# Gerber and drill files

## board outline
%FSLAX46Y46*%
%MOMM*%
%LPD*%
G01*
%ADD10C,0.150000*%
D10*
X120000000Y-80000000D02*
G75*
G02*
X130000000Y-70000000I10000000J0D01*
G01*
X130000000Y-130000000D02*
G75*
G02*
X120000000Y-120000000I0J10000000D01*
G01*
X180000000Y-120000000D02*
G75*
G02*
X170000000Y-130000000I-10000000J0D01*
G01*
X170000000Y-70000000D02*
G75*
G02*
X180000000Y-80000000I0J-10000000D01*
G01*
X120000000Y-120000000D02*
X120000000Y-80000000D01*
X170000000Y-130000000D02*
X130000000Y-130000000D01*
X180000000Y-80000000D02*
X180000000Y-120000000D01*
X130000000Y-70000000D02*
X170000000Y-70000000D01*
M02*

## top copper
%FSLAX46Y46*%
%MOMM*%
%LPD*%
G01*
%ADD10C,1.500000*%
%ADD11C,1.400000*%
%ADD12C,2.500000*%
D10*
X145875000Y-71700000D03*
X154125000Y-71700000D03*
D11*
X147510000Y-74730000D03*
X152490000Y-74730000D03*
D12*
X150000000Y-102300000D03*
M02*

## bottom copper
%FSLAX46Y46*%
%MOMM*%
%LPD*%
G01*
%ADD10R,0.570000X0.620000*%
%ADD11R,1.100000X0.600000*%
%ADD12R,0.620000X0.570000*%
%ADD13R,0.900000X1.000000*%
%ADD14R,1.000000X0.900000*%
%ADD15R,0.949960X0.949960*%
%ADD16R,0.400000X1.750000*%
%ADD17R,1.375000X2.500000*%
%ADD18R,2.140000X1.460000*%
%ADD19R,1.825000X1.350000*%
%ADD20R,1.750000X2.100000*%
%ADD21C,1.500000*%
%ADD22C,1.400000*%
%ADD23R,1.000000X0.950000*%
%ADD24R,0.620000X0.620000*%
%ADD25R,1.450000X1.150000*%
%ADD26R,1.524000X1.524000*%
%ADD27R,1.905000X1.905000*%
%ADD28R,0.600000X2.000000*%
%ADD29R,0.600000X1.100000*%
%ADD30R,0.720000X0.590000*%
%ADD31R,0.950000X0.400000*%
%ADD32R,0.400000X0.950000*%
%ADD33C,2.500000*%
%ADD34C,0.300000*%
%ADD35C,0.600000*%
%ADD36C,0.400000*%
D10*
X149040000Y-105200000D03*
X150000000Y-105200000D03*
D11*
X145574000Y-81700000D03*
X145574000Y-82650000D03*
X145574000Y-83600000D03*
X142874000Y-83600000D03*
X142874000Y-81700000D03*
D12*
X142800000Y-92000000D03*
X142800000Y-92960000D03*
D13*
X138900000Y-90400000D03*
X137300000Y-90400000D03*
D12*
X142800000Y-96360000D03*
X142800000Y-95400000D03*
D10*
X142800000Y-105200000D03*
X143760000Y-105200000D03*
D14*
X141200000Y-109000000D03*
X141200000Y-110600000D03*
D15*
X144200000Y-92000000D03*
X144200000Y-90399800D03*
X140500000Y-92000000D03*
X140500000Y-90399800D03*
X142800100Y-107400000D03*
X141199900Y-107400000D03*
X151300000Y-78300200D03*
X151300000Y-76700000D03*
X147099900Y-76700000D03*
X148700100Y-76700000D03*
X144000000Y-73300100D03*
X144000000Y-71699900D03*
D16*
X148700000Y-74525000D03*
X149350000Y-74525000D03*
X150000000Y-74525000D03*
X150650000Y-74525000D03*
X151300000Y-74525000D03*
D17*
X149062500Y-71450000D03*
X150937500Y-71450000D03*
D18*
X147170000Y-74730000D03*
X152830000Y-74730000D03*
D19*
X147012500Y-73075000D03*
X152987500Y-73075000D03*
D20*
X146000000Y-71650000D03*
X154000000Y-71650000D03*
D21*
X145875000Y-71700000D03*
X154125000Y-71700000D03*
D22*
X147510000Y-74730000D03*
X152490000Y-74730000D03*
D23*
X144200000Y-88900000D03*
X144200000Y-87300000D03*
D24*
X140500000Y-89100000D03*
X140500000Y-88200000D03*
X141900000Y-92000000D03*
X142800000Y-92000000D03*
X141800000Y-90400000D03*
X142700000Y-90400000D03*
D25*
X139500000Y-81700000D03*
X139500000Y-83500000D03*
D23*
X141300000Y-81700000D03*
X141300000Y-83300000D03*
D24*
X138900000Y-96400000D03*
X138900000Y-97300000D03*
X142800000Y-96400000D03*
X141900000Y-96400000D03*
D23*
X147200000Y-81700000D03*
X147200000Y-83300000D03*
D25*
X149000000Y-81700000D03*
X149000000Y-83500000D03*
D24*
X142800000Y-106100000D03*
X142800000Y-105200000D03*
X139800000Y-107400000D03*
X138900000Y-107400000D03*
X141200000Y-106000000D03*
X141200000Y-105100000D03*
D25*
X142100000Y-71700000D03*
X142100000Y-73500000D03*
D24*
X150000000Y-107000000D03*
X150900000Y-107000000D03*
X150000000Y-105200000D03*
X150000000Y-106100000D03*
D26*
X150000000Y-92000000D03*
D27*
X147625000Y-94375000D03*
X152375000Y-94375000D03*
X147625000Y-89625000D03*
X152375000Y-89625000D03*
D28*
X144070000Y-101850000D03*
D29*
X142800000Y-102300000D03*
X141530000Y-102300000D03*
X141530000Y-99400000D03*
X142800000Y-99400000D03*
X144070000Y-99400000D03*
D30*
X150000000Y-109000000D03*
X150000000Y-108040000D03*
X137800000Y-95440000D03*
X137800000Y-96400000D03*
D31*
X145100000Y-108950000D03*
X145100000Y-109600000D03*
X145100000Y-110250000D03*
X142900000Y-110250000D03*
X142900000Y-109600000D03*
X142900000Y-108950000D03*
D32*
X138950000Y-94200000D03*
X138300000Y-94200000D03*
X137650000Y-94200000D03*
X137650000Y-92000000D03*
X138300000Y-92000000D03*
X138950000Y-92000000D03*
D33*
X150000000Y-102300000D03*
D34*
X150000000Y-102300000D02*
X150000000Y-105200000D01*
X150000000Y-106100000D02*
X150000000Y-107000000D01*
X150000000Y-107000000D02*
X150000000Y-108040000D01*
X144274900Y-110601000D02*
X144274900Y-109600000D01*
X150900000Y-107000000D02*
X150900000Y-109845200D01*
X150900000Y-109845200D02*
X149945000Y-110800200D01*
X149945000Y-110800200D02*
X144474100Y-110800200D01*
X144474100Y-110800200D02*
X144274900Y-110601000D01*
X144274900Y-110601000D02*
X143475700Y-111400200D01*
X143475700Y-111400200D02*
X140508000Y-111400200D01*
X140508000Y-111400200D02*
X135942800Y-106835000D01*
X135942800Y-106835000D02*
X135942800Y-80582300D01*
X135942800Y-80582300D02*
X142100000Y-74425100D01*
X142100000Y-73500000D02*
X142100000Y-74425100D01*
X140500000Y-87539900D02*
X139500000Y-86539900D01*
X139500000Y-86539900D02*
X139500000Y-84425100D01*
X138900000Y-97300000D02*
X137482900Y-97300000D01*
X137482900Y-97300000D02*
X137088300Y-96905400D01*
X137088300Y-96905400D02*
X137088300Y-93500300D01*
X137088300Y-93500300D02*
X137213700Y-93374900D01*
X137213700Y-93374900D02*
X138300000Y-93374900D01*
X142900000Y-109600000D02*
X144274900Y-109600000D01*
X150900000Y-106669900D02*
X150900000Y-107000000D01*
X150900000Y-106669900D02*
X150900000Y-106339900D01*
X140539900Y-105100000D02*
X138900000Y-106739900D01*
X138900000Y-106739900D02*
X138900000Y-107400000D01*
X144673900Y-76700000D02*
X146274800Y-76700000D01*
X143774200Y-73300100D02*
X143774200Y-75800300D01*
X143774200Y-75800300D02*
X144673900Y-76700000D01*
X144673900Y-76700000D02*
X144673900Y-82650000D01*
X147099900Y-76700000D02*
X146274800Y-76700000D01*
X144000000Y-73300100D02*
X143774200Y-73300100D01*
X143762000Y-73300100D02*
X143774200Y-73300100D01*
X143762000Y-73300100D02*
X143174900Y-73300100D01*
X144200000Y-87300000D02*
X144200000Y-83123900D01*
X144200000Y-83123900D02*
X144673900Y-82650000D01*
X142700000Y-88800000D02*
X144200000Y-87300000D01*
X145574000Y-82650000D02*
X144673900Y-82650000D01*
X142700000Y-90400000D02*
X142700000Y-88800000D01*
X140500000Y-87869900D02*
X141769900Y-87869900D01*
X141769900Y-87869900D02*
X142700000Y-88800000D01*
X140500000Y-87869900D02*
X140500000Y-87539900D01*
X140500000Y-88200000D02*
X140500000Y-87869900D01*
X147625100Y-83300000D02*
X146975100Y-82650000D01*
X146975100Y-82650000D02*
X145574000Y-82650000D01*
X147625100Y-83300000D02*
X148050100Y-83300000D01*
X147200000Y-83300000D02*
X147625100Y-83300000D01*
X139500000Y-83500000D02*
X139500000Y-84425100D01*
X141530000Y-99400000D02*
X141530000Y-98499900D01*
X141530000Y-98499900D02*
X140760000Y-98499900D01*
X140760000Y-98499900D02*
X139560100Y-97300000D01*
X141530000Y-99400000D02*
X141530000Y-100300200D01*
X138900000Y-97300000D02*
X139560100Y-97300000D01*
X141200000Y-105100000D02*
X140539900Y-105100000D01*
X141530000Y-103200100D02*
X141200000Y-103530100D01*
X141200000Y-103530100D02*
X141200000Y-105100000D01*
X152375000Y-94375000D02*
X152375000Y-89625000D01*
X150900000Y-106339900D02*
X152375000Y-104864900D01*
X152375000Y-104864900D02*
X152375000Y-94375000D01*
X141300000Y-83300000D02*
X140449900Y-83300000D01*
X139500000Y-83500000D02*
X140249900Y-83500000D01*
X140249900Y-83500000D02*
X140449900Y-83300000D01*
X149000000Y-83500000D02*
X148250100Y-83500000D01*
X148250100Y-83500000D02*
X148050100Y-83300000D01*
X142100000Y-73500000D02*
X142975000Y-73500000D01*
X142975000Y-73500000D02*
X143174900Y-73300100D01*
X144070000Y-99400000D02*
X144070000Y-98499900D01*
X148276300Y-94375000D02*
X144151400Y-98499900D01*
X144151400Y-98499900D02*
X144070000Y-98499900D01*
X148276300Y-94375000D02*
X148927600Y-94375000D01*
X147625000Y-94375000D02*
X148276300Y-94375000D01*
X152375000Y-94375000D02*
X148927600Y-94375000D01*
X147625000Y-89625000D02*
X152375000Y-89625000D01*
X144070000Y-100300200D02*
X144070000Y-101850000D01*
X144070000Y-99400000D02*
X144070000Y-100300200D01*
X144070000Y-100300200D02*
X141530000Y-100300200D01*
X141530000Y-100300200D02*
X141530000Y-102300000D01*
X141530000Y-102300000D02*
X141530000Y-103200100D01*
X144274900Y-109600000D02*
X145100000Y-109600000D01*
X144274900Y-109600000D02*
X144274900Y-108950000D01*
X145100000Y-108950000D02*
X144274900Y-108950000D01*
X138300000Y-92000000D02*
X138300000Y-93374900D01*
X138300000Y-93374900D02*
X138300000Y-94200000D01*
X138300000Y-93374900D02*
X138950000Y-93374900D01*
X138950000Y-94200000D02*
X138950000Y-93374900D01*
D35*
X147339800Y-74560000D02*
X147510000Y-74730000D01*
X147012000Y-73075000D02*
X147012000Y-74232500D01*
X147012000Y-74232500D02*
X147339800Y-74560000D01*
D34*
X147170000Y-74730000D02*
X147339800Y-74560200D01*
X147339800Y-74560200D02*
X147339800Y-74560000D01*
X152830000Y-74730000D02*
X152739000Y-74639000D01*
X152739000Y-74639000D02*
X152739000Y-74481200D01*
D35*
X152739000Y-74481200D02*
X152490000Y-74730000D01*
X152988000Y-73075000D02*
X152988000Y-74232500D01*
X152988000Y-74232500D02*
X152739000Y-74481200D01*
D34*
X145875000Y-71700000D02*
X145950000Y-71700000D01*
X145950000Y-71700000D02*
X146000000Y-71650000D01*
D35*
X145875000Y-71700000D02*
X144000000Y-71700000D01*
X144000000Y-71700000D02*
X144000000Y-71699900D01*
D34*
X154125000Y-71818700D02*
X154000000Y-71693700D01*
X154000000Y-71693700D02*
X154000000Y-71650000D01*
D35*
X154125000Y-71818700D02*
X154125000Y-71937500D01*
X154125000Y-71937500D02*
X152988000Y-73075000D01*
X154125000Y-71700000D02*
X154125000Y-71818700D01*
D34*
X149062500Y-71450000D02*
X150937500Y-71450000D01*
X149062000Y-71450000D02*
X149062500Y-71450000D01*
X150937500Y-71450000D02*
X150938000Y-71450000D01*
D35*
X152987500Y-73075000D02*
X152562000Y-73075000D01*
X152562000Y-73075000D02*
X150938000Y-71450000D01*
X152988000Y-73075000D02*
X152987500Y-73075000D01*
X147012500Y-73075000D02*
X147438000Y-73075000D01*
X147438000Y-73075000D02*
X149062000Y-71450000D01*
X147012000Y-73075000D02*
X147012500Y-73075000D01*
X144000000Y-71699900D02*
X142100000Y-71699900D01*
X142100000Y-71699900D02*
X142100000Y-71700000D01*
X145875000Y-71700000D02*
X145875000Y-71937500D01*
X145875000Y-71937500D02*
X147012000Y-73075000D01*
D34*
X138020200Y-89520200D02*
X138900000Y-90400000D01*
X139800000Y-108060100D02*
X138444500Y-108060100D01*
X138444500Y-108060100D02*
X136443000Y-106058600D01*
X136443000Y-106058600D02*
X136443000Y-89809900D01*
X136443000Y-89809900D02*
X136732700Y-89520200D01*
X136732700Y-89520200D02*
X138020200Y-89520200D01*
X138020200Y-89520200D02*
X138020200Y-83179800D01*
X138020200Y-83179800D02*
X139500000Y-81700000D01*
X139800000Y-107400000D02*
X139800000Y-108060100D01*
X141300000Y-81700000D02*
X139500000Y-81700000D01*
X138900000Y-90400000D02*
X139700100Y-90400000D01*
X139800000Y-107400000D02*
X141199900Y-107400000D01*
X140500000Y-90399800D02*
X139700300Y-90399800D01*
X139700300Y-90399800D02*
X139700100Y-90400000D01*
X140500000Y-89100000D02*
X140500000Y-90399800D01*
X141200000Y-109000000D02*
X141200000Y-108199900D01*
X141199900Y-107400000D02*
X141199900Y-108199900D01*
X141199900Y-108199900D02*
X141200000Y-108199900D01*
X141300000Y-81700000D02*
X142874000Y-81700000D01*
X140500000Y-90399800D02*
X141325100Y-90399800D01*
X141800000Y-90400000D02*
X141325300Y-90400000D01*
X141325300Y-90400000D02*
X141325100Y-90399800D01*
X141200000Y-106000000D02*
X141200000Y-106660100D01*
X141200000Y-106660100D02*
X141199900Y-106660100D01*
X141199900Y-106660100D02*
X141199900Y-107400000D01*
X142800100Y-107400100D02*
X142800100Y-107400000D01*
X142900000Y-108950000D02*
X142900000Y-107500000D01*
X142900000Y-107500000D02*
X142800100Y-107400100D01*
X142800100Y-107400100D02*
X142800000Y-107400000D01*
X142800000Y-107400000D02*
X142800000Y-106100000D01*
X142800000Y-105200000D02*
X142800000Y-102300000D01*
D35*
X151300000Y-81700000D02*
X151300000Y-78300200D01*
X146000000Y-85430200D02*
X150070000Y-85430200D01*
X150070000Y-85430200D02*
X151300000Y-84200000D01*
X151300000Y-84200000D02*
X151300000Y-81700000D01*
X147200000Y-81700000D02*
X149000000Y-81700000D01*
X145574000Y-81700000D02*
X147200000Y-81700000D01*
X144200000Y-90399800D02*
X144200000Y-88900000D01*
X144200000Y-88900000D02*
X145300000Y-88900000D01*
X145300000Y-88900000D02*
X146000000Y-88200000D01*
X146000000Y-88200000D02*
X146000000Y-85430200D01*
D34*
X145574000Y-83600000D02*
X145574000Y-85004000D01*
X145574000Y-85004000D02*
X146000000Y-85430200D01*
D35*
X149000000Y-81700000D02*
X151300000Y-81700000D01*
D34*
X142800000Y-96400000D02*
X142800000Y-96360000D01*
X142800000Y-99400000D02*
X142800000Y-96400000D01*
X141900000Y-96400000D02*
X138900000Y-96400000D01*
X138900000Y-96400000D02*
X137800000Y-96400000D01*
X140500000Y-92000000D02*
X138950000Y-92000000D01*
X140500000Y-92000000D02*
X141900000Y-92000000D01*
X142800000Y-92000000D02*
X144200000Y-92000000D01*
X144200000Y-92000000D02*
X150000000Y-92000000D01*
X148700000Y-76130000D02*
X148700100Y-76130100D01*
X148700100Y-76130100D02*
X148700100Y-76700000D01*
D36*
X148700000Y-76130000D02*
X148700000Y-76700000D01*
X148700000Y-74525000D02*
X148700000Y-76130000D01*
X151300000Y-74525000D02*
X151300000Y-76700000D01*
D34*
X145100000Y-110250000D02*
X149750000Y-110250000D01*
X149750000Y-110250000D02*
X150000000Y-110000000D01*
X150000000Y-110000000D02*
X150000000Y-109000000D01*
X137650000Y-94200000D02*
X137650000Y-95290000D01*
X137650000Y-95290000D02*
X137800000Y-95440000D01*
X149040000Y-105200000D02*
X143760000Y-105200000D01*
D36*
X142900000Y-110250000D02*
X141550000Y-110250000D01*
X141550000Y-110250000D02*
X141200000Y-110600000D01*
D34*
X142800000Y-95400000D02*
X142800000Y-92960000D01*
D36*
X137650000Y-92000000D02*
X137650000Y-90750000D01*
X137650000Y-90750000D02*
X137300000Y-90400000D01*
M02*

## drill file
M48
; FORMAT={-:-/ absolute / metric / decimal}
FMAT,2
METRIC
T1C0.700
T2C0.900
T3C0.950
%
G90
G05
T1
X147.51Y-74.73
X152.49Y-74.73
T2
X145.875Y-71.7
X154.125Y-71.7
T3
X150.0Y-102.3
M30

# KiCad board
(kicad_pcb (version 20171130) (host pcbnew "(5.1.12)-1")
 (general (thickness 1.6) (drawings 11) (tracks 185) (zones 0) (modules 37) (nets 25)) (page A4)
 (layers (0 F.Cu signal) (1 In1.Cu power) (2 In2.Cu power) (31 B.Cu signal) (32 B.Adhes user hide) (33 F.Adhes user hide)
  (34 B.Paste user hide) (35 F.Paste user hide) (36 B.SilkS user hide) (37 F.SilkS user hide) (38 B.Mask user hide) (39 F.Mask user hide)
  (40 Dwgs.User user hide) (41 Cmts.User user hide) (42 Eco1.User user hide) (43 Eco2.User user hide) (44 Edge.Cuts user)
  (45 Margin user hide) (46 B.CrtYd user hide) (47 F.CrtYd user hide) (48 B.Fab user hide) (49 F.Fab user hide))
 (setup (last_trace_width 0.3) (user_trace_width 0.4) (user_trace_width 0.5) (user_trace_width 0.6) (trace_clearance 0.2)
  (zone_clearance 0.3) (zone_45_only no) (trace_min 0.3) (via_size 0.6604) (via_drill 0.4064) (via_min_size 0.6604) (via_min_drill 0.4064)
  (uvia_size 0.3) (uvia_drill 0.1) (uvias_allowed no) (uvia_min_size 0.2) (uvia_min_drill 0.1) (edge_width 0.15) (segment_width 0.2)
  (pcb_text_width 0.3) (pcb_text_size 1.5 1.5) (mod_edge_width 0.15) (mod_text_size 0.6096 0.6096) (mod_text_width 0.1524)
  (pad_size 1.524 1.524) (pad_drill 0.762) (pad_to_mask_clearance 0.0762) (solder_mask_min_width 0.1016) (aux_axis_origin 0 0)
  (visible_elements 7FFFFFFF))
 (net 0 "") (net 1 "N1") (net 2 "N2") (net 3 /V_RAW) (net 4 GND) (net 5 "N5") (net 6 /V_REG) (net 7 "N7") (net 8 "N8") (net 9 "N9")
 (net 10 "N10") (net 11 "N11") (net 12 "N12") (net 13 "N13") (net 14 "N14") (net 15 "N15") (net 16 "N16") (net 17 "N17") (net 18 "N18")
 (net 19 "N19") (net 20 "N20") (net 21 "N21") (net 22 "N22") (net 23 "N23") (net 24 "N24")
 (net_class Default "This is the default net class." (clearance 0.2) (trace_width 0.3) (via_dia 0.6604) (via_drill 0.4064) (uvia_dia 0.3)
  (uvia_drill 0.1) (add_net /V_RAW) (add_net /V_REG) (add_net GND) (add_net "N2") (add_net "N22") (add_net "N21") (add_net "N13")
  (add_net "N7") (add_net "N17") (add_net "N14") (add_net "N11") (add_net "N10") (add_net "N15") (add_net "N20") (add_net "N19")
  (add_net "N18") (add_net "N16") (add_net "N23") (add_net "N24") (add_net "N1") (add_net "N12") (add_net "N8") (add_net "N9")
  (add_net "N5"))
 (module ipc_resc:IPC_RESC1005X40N (layer B.Cu) (at 149.52 105.2)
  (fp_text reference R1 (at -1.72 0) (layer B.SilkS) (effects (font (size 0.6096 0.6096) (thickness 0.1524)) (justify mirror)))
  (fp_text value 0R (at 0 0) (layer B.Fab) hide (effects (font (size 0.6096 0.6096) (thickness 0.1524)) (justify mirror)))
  (pad 1 smd rect (at -0.48 0) (size 0.57 0.62) (layers B.Cu B.Paste B.Mask) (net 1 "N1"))
  (pad 2 smd rect (at 0.48 0) (size 0.57 0.62) (layers B.Cu B.Paste B.Mask) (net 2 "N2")))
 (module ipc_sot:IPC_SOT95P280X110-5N (layer B.Cu) (at 144.224 82.65 180)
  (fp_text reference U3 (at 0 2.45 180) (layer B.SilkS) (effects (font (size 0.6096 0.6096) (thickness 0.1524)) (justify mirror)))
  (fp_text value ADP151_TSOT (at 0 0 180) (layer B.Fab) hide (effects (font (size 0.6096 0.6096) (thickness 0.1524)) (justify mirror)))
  (pad 1 smd rect (at -1.35 0.95 180) (size 1.1 0.6) (layers B.Cu B.Paste B.Mask) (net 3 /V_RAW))
  (pad 2 smd rect (at -1.35 0 180) (size 1.1 0.6) (layers B.Cu B.Paste B.Mask) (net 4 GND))
  (pad 3 smd rect (at -1.35 -0.95 180) (size 1.1 0.6) (layers B.Cu B.Paste B.Mask) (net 3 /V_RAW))
  (pad 4 smd rect (at 1.35 -0.95 180) (size 1.1 0.6) (layers B.Cu B.Paste B.Mask) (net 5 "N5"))
  (pad 5 smd rect (at 1.35 0.95 180) (size 1.1 0.6) (layers B.Cu B.Paste B.Mask) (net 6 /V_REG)))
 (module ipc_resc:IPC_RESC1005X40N (layer B.Cu) (at 142.8 92.48 270)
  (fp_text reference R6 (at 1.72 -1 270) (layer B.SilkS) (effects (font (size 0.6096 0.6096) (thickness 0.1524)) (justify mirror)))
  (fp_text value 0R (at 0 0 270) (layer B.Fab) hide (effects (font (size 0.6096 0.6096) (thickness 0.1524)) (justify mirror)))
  (pad 1 smd rect (at -0.48 0 270) (size 0.57 0.62) (layers B.Cu B.Paste B.Mask) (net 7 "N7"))
  (pad 2 smd rect (at 0.48 0 270) (size 0.57 0.62) (layers B.Cu B.Paste B.Mask) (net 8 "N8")))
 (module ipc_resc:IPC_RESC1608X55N (layer B.Cu) (at 138.1 90.4 180)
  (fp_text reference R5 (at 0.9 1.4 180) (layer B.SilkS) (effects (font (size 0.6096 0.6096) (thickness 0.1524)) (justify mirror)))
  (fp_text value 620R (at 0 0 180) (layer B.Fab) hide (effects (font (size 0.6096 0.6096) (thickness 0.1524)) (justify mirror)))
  (pad 1 smd rect (at -0.8 0 180) (size 0.9 1) (layers B.Cu B.Paste B.Mask) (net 6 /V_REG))
  (pad 2 smd rect (at 0.8 0 180) (size 0.9 1) (layers B.Cu B.Paste B.Mask) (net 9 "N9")))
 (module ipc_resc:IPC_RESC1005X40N (layer B.Cu) (at 142.8 95.88 90)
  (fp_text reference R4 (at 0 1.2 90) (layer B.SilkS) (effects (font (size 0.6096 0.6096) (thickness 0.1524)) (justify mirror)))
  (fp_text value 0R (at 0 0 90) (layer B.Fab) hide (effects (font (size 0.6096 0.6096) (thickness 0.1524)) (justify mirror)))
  (pad 1 smd rect (at -0.48 0 90) (size 0.57 0.62) (layers B.Cu B.Paste B.Mask) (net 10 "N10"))
  (pad 2 smd rect (at 0.48 0 90) (size 0.57 0.62) (layers B.Cu B.Paste B.Mask) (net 8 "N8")))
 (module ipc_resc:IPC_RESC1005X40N (layer B.Cu) (at 143.28 105.2)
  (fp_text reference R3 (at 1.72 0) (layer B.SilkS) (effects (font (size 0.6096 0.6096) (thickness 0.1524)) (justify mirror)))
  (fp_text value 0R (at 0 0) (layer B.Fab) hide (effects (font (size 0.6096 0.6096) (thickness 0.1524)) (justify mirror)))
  (pad 1 smd rect (at -0.48 0) (size 0.57 0.62) (layers B.Cu B.Paste B.Mask) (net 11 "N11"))
  (pad 2 smd rect (at 0.48 0) (size 0.57 0.62) (layers B.Cu B.Paste B.Mask) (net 1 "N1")))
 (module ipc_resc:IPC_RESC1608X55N (layer B.Cu) (at 141.2 109.8 270)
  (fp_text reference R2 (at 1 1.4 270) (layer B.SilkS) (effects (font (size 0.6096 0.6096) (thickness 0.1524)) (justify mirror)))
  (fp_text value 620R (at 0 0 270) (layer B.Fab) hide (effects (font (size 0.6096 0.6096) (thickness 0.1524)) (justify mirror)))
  (pad 1 smd rect (at -0.8 0 270) (size 0.9 1) (layers B.Cu B.Paste B.Mask) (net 6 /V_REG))
  (pad 2 smd rect (at 0.8 0 270) (size 0.9 1) (layers B.Cu B.Paste B.Mask) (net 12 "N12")))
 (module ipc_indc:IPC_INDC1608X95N (layer B.Cu) (at 144.2 91.1999 90)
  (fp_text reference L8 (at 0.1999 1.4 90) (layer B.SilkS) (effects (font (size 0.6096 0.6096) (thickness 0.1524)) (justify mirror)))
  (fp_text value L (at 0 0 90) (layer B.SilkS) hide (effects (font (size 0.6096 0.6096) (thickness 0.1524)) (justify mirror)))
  (pad 1 smd rect (at -0.8001 0 90) (size 0.94996 0.94996) (layers B.Cu B.Paste B.Mask) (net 7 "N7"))
  (pad 2 smd rect (at 0.8001 0 90) (size 0.94996 0.94996) (layers B.Cu B.Paste B.Mask) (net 3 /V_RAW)))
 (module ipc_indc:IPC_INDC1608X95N (layer B.Cu) (at 140.5 91.1999 90)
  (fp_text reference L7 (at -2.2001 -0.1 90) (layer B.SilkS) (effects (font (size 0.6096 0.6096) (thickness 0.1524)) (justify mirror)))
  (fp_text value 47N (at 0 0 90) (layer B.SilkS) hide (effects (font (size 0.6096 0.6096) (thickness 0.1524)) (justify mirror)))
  (pad 1 smd rect (at -0.8001 0 90) (size 0.94996 0.94996) (layers B.Cu B.Paste B.Mask) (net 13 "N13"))
  (pad 2 smd rect (at 0.8001 0 90) (size 0.94996 0.94996) (layers B.Cu B.Paste B.Mask) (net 6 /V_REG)))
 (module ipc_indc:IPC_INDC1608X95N (layer B.Cu) (at 142 107.4 180)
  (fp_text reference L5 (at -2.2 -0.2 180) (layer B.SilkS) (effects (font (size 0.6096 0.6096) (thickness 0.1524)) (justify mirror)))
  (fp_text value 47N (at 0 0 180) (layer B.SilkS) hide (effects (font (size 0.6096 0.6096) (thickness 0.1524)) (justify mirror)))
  (pad 1 smd rect (at -0.8001 0 180) (size 0.94996 0.94996) (layers B.Cu B.Paste B.Mask) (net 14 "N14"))
  (pad 2 smd rect (at 0.8001 0 180) (size 0.94996 0.94996) (layers B.Cu B.Paste B.Mask) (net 6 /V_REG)))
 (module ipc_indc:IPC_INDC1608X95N (layer B.Cu) (at 151.3 77.5001 90)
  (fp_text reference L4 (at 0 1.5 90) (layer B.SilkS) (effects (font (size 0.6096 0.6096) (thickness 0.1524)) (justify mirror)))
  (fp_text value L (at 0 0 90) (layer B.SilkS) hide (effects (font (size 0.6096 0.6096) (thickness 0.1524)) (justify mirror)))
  (pad 1 smd rect (at -0.8001 0 90) (size 0.94996 0.94996) (layers B.Cu B.Paste B.Mask) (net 3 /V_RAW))
  (pad 2 smd rect (at 0.8001 0 90) (size 0.94996 0.94996) (layers B.Cu B.Paste B.Mask) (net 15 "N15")))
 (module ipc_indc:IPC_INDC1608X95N (layer B.Cu) (at 147.9 76.7)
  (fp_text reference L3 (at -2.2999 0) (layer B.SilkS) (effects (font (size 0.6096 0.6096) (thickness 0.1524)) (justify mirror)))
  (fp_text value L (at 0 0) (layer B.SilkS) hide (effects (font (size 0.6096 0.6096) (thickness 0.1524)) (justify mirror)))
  (pad 1 smd rect (at -0.8001 0) (size 0.94996 0.94996) (layers B.Cu B.Paste B.Mask) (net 4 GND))
  (pad 2 smd rect (at 0.8001 0) (size 0.94996 0.94996) (layers B.Cu B.Paste B.Mask) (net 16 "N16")))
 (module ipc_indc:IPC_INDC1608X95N (layer B.Cu) (at 144 72.5 90)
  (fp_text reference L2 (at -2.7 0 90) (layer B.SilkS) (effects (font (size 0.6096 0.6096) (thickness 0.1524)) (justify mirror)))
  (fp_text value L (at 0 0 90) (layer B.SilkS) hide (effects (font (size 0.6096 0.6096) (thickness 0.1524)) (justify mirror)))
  (pad 1 smd rect (at -0.8001 0 90) (size 0.94996 0.94996) (layers B.Cu B.Paste B.Mask) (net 4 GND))
  (pad 2 smd rect (at 0.8001 0 90) (size 0.94996 0.94996) (layers B.Cu B.Paste B.Mask) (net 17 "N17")))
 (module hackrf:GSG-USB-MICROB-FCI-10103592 (layer B.Cu) (at 150 70 270)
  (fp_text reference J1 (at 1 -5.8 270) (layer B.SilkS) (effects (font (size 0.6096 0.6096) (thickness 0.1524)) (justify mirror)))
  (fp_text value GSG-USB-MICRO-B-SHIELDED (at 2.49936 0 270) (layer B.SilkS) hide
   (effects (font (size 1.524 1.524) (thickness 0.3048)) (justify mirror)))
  (pad 5 smd rect (at 4.525 1.3 270) (size 1.75 0.4) (layers B.Cu B.Paste B.Mask) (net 16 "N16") (solder_mask_margin 0.1016)
   (clearance 0.2032))
  (pad 4 smd rect (at 4.525 0.65 270) (size 1.75 0.4) (layers B.Cu B.Paste B.Mask) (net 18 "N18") (solder_mask_margin 0.1016)
   (clearance 0.2032))
  (pad 3 smd rect (at 4.525 0 270) (size 1.75 0.4) (layers B.Cu B.Paste B.Mask) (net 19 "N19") (solder_mask_margin 0.1016)
   (clearance 0.2032))
  (pad 2 smd rect (at 4.525 -0.65 270) (size 1.75 0.4) (layers B.Cu B.Paste B.Mask) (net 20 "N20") (solder_mask_margin 0.1016)
   (clearance 0.2032))
  (pad 1 smd rect (at 4.525 -1.3 270) (size 1.75 0.4) (layers B.Cu B.Paste B.Mask) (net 15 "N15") (solder_mask_margin 0.1016)
   (clearance 0.2032))
  (pad 0 smd rect (at 1.45 0.9375 270) (size 2.5 1.375) (layers B.Cu B.Paste B.Mask) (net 17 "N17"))
  (pad 0 smd rect (at 1.45 -0.9375 270) (size 2.5 1.375) (layers B.Cu B.Paste B.Mask) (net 17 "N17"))
  (pad 0 smd rect (at 4.73 2.83 270) (size 1.46 2.14) (layers B.Cu B.Paste B.Mask) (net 17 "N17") (solder_paste_margin_ratio -0.05))
  (pad 0 smd rect (at 4.73 -2.83 270) (size 1.46 2.14) (layers B.Cu B.Paste B.Mask) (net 17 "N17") (solder_paste_margin_ratio -0.05))
  (pad 0 smd rect (at 3.075 2.9875 270) (size 1.35 1.825) (layers B.Cu B.Mask) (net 17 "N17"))
  (pad 0 smd rect (at 3.075 -2.9875 270) (size 1.35 1.825) (layers B.Cu B.Mask) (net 17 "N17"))
  (pad 0 smd rect (at 1.65 4 270) (size 2.1 1.75) (layers B.Cu B.Paste B.Mask) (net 17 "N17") (solder_paste_margin_ratio -0.05))
  (pad 0 smd rect (at 1.65 -4 270) (size 2.1 1.75) (layers B.Cu B.Paste B.Mask) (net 17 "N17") (solder_paste_margin_ratio -0.05))
  (pad 0 thru_hole circle (at 1.7 4.125 270) (size 1.5 1.5) (drill 0.9) (layers *.Cu *.Mask) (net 17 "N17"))
  (pad 0 thru_hole circle (at 1.7 -4.125 270) (size 1.5 1.5) (drill 0.9) (layers *.Cu *.Mask) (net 17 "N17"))
  (pad 0 thru_hole circle (at 4.73 2.49 270) (size 1.4 1.4) (drill 0.7) (layers *.Cu *.Mask) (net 17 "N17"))
  (pad 0 thru_hole circle (at 4.73 -2.49 270) (size 1.4 1.4) (drill 0.7) (layers *.Cu *.Mask) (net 17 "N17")))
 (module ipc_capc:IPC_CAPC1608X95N (layer B.Cu) (at 144.2 88.1 90)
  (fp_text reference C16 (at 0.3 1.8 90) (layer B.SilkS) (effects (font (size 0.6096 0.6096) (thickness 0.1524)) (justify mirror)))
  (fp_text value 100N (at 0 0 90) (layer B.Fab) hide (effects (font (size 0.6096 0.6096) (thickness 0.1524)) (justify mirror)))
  (pad 1 smd rect (at -0.8 0 90) (size 0.95 1) (layers B.Cu B.Paste B.Mask) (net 3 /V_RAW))
  (pad 2 smd rect (at 0.8 0 90) (size 0.95 1) (layers B.Cu B.Paste B.Mask) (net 4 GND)))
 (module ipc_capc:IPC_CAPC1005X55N (layer B.Cu) (at 140.5 88.65 90)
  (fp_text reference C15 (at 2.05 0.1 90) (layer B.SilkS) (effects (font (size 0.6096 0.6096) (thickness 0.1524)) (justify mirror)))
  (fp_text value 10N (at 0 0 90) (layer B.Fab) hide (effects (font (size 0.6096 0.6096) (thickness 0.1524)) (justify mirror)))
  (pad 1 smd rect (at -0.45 0 90) (size 0.62 0.62) (layers B.Cu B.Paste B.Mask) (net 6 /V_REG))
  (pad 2 smd rect (at 0.45 0 90) (size 0.62 0.62) (layers B.Cu B.Paste B.Mask) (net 4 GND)))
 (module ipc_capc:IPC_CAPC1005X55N (layer B.Cu) (at 142.35 92)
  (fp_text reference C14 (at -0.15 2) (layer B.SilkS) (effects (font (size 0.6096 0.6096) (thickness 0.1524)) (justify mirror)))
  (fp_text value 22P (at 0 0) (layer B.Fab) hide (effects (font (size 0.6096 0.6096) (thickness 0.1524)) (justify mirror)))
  (pad 1 smd rect (at -0.45 0) (size 0.62 0.62) (layers B.Cu B.Paste B.Mask) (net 13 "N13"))
  (pad 2 smd rect (at 0.45 0) (size 0.62 0.62) (layers B.Cu B.Paste B.Mask) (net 7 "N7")))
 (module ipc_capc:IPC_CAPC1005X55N (layer B.Cu) (at 142.25 90.4)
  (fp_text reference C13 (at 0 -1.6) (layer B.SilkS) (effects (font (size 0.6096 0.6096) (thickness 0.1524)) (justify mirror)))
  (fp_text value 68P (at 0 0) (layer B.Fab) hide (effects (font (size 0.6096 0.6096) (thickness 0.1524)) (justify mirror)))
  (pad 1 smd rect (at -0.45 0) (size 0.62 0.62) (layers B.Cu B.Paste B.Mask) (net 6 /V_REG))
  (pad 2 smd rect (at 0.45 0) (size 0.62 0.62) (layers B.Cu B.Paste B.Mask) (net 4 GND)))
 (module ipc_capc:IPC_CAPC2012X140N (layer B.Cu) (at 139.5 82.6 270)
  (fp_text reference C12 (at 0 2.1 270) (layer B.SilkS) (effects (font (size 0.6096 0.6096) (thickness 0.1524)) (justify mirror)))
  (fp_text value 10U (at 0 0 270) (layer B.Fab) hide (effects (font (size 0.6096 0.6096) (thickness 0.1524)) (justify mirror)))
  (pad 1 smd rect (at -0.9 0 270) (size 1.15 1.45) (layers B.Cu B.Paste B.Mask) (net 6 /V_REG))
  (pad 2 smd rect (at 0.9 0 270) (size 1.15 1.45) (layers B.Cu B.Paste B.Mask) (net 4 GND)))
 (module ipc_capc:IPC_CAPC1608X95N (layer B.Cu) (at 141.3 82.5 270)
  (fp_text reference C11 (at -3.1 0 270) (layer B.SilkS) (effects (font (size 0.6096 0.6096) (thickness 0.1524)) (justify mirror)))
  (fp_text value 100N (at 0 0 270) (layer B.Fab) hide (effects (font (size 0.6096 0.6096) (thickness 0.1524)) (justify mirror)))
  (pad 1 smd rect (at -0.8 0 270) (size 0.95 1) (layers B.Cu B.Paste B.Mask) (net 6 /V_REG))
  (pad 2 smd rect (at 0.8 0 270) (size 0.95 1) (layers B.Cu B.Paste B.Mask) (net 4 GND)))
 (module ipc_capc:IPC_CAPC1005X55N (layer B.Cu) (at 138.9 96.85 270)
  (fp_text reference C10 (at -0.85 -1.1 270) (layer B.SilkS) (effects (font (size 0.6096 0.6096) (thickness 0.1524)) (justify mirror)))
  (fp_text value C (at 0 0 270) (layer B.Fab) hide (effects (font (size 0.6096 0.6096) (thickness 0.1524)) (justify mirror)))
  (pad 1 smd rect (at -0.45 0 270) (size 0.62 0.62) (layers B.Cu B.Paste B.Mask) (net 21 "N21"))
  (pad 2 smd rect (at 0.45 0 270) (size 0.62 0.62) (layers B.Cu B.Paste B.Mask) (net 4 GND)))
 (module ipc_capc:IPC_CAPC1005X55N (layer B.Cu) (at 142.35 96.4 180)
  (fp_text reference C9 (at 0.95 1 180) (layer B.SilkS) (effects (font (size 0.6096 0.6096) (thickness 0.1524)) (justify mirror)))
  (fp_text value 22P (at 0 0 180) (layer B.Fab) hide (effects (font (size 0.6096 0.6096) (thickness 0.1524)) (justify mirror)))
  (pad 1 smd rect (at -0.45 0 180) (size 0.62 0.62) (layers B.Cu B.Paste B.Mask) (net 10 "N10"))
  (pad 2 smd rect (at 0.45 0 180) (size 0.62 0.62) (layers B.Cu B.Paste B.Mask) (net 21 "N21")))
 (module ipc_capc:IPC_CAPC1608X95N (layer B.Cu) (at 147.2 82.5 270)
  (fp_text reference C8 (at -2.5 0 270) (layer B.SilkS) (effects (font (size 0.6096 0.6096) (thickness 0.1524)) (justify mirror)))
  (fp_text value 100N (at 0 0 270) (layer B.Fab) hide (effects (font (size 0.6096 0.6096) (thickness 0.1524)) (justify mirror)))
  (pad 1 smd rect (at -0.8 0 270) (size 0.95 1) (layers B.Cu B.Paste B.Mask) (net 3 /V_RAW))
  (pad 2 smd rect (at 0.8 0 270) (size 0.95 1) (layers B.Cu B.Paste B.Mask) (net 4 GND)))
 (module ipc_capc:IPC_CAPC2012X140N (layer B.Cu) (at 149 82.6 270)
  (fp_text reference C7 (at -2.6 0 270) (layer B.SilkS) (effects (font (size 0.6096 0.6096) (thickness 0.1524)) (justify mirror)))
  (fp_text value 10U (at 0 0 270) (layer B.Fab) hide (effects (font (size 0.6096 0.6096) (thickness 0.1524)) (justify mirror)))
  (pad 1 smd rect (at -0.9 0 270) (size 1.15 1.45) (layers B.Cu B.Paste B.Mask) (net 3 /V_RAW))
  (pad 2 smd rect (at 0.9 0 270) (size 1.15 1.45) (layers B.Cu B.Paste B.Mask) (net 4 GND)))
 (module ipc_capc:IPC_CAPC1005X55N (layer B.Cu) (at 142.8 105.65 90)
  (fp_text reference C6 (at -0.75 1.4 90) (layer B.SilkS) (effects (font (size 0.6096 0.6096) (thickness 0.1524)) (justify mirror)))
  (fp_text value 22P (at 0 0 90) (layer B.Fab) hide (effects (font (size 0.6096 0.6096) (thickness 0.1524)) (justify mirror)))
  (pad 1 smd rect (at -0.45 0 90) (size 0.62 0.62) (layers B.Cu B.Paste B.Mask) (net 14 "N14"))
  (pad 2 smd rect (at 0.45 0 90) (size 0.62 0.62) (layers B.Cu B.Paste B.Mask) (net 11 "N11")))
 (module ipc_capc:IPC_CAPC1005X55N (layer B.Cu) (at 139.35 107.4 180)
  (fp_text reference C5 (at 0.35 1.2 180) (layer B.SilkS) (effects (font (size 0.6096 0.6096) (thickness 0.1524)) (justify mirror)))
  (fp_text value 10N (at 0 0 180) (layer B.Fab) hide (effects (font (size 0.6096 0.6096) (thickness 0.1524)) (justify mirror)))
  (pad 1 smd rect (at -0.45 0 180) (size 0.62 0.62) (layers B.Cu B.Paste B.Mask) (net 6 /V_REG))
  (pad 2 smd rect (at 0.45 0 180) (size 0.62 0.62) (layers B.Cu B.Paste B.Mask) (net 4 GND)))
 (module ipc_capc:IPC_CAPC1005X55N (layer B.Cu) (at 141.2 105.55 90)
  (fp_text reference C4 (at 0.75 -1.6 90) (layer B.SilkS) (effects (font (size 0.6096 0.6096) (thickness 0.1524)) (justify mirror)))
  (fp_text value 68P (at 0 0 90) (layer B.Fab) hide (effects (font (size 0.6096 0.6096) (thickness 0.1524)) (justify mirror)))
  (pad 1 smd rect (at -0.45 0 90) (size 0.62 0.62) (layers B.Cu B.Paste B.Mask) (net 6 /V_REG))
  (pad 2 smd rect (at 0.45 0 90) (size 0.62 0.62) (layers B.Cu B.Paste B.Mask) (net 4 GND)))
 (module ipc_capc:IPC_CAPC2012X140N (layer B.Cu) (at 142.1 72.6 270)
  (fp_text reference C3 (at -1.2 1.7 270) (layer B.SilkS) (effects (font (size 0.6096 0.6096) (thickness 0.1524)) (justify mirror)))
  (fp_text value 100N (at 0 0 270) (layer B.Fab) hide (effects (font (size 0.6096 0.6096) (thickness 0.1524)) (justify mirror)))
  (pad 1 smd rect (at -0.9 0 270) (size 1.15 1.45) (layers B.Cu B.Paste B.Mask) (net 17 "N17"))
  (pad 2 smd rect (at 0.9 0 270) (size 1.15 1.45) (layers B.Cu B.Paste B.Mask) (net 4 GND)))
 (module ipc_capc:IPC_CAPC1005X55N (layer B.Cu) (at 150.45 107)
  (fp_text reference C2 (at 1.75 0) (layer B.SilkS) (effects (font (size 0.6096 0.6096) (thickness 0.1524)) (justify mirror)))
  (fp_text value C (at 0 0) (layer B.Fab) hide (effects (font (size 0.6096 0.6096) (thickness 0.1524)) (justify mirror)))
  (pad 1 smd rect (at -0.45 0) (size 0.62 0.62) (layers B.Cu B.Paste B.Mask) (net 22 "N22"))
  (pad 2 smd rect (at 0.45 0) (size 0.62 0.62) (layers B.Cu B.Paste B.Mask) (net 4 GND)))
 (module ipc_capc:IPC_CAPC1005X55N (layer B.Cu) (at 150 105.65 270)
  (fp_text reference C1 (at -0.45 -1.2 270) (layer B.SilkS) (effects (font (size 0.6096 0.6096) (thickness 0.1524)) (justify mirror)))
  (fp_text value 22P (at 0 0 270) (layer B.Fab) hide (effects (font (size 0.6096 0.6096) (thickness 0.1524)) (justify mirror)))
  (pad 1 smd rect (at -0.45 0 270) (size 0.62 0.62) (layers B.Cu B.Paste B.Mask) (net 2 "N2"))
  (pad 2 smd rect (at 0.45 0 270) (size 0.62 0.62) (layers B.Cu B.Paste B.Mask) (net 22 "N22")))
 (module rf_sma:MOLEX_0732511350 (layer B.Cu) (at 150 92)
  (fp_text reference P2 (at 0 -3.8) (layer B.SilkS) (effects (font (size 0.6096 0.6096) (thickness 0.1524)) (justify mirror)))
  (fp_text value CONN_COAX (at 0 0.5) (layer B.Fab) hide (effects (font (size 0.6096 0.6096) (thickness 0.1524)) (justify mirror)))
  (pad 1 smd rect (at 0 0) (size 1.524 1.524) (layers B.Cu B.Paste B.Mask) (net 7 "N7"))
  (pad 2 smd rect (at -2.375 2.375) (size 1.905 1.905) (layers B.Cu B.Paste B.Mask) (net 4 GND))
  (pad 2 smd rect (at 2.375 2.375) (size 1.905 1.905) (layers B.Cu B.Paste B.Mask) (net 4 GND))
  (pad 2 smd rect (at -2.375 -2.375) (size 1.905 1.905) (layers B.Cu B.Paste B.Mask) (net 4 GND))
  (pad 2 smd rect (at 2.375 -2.375) (size 1.905 1.905) (layers B.Cu B.Paste B.Mask) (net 4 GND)))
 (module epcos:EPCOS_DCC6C (layer B.Cu) (at 142.8 100.85 90)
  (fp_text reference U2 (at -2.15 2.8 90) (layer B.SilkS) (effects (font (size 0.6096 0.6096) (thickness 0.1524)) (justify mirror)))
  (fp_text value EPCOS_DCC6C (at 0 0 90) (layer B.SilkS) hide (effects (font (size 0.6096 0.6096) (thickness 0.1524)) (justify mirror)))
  (pad 1 smd rect (at -1 1.27 90) (size 2 0.6) (layers B.Cu B.Paste B.Mask) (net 4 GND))
  (pad 2 smd rect (at -1.45 0 90) (size 1.1 0.6) (layers B.Cu B.Paste B.Mask) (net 11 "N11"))
  (pad 3 smd rect (at -1.45 -1.27 90) (size 1.1 0.6) (layers B.Cu B.Paste B.Mask) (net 4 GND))
  (pad 4 smd rect (at 1.45 -1.27 90) (size 1.1 0.6) (layers B.Cu B.Paste B.Mask) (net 4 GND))
  (pad 5 smd rect (at 1.45 0 90) (size 1.1 0.6) (layers B.Cu B.Paste B.Mask) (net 10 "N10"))
  (pad 6 smd rect (at 1.45 1.27 90) (size 1.1 0.6) (layers B.Cu B.Paste B.Mask) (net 4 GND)))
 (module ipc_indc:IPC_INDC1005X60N (layer B.Cu) (at 150 108.52 90)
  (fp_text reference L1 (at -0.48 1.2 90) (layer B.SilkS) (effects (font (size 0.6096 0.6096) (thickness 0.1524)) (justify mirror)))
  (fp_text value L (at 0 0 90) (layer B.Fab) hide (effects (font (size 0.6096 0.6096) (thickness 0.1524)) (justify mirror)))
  (pad 1 smd rect (at -0.48 0 90) (size 0.59 0.72) (layers B.Cu B.Paste B.Mask) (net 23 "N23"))
  (pad 2 smd rect (at 0.48 0 90) (size 0.59 0.72) (layers B.Cu B.Paste B.Mask) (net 22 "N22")))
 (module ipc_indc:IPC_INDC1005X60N (layer B.Cu) (at 137.8 95.92 270)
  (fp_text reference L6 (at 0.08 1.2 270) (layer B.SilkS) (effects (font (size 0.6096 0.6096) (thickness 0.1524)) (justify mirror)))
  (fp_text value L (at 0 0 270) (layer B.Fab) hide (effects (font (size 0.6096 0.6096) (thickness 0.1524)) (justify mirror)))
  (pad 1 smd rect (at -0.48 0 270) (size 0.59 0.72) (layers B.Cu B.Paste B.Mask) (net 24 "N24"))
  (pad 2 smd rect (at 0.48 0 270) (size 0.59 0.72) (layers B.Cu B.Paste B.Mask) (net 21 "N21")))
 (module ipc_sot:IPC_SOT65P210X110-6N (layer B.Cu) (at 144 109.6 180)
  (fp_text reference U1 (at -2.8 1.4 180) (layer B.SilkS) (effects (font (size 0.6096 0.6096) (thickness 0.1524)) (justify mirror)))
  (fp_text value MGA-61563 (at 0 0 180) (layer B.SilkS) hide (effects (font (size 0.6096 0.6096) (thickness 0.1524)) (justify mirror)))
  (pad 1 smd rect (at -1.1 0.65 180) (size 0.95 0.4) (layers B.Cu B.Paste B.Mask) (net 4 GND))
  (pad 2 smd rect (at -1.1 0 180) (size 0.95 0.4) (layers B.Cu B.Paste B.Mask) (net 4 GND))
  (pad 3 smd rect (at -1.1 -0.65 180) (size 0.95 0.4) (layers B.Cu B.Paste B.Mask) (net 23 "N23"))
  (pad 4 smd rect (at 1.1 -0.65 180) (size 0.95 0.4) (layers B.Cu B.Paste B.Mask) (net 12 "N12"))
  (pad 5 smd rect (at 1.1 0 180) (size 0.95 0.4) (layers B.Cu B.Paste B.Mask) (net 4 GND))
  (pad 6 smd rect (at 1.1 0.65 180) (size 0.95 0.4) (layers B.Cu B.Paste B.Mask) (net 14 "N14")))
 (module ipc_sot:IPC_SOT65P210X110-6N (layer B.Cu) (at 138.3 93.1 90)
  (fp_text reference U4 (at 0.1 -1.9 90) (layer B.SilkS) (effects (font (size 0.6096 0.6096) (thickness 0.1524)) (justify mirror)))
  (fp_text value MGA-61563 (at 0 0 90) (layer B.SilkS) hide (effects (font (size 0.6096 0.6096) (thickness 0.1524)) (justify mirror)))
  (pad 1 smd rect (at -1.1 0.65 90) (size 0.95 0.4) (layers B.Cu B.Paste B.Mask) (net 4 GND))
  (pad 2 smd rect (at -1.1 0 90) (size 0.95 0.4) (layers B.Cu B.Paste B.Mask) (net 4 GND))
  (pad 3 smd rect (at -1.1 -0.65 90) (size 0.95 0.4) (layers B.Cu B.Paste B.Mask) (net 24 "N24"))
  (pad 4 smd rect (at 1.1 -0.65 90) (size 0.95 0.4) (layers B.Cu B.Paste B.Mask) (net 9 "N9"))
  (pad 5 smd rect (at 1.1 0 90) (size 0.95 0.4) (layers B.Cu B.Paste B.Mask) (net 4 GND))
  (pad 6 smd rect (at 1.1 0.65 90) (size 0.95 0.4) (layers B.Cu B.Paste B.Mask) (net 13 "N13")))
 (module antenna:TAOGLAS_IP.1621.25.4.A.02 (layer F.Cu) (at 150 100)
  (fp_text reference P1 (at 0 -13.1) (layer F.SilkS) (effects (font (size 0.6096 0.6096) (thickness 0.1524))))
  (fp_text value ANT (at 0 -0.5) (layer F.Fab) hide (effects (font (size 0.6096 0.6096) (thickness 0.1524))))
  (pad 1 thru_hole circle (at 0 2.3) (size 2.5 2.5) (drill 0.95) (layers B.Cu) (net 2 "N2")))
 (gr_arc (start 130 80) (end 120 80) (angle 90) (layer Edge.Cuts) (width 0.15))
 (gr_arc (start 130 120) (end 130 130) (angle 90) (layer Edge.Cuts) (width 0.15))
 (gr_arc (start 170 120) (end 180 120) (angle 90) (layer Edge.Cuts) (width 0.15))
 (gr_arc (start 170 80) (end 170 70) (angle 90) (layer Edge.Cuts) (width 0.15))
 (gr_line (start 120 120) (end 120 80) (layer Edge.Cuts) (width 0.15))
 (gr_line (start 170 130) (end 130 130) (layer Edge.Cuts) (width 0.15))
 (gr_line (start 180 80) (end 180 120) (layer Edge.Cuts) (width 0.15))
 (gr_line (start 130 70) (end 170 70) (layer Edge.Cuts) (width 0.15))
 (segment (start 150 102.3) (end 150 105.2) (width 0.3) (layer B.Cu) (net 2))
 (segment (start 150 106.1) (end 150 107) (width 0.3) (layer B.Cu) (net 22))
 (segment (start 150 107) (end 150 108.04) (width 0.3) (layer B.Cu) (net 22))
 (segment (start 144.2749 110.601) (end 144.2749 109.6) (width 0.3) (layer B.Cu) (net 4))
 (segment (start 150.9 107) (end 150.9 109.8452) (width 0.3) (layer B.Cu) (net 4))
 (segment (start 150.9 109.8452) (end 149.945 110.8002) (width 0.3) (layer B.Cu) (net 4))
 (segment (start 149.945 110.8002) (end 144.4741 110.8002) (width 0.3) (layer B.Cu) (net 4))
 (segment (start 144.4741 110.8002) (end 144.2749 110.601) (width 0.3) (layer B.Cu) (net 4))
 (segment (start 144.2749 110.601) (end 143.4757 111.4002) (width 0.3) (layer B.Cu) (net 4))
 (segment (start 143.4757 111.4002) (end 140.508 111.4002) (width 0.3) (layer B.Cu) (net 4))
 (segment (start 140.508 111.4002) (end 135.9428 106.835) (width 0.3) (layer B.Cu) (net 4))
 (segment (start 135.9428 106.835) (end 135.9428 80.5823) (width 0.3) (layer B.Cu) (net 4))
 (segment (start 135.9428 80.5823) (end 142.1 74.4251) (width 0.3) (layer B.Cu) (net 4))
 (segment (start 142.1 73.5) (end 142.1 74.4251) (width 0.3) (layer B.Cu) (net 4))
 (segment (start 140.5 87.5399) (end 139.5 86.5399) (width 0.3) (layer B.Cu) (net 4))
 (segment (start 139.5 86.5399) (end 139.5 84.4251) (width 0.3) (layer B.Cu) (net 4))
 (segment (start 138.9 97.3) (end 137.4829 97.3) (width 0.3) (layer B.Cu) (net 4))
 (segment (start 137.4829 97.3) (end 137.0883 96.9054) (width 0.3) (layer B.Cu) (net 4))
 (segment (start 137.0883 96.9054) (end 137.0883 93.5003) (width 0.3) (layer B.Cu) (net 4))
 (segment (start 137.0883 93.5003) (end 137.2137 93.3749) (width 0.3) (layer B.Cu) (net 4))
 (segment (start 137.2137 93.3749) (end 138.3 93.3749) (width 0.3) (layer B.Cu) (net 4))
 (segment (start 142.9 109.6) (end 144.2749 109.6) (width 0.3) (layer B.Cu) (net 4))
 (segment (start 150.9 106.6699) (end 150.9 107) (width 0.3) (layer B.Cu) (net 4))
 (segment (start 150.9 106.6699) (end 150.9 106.3399) (width 0.3) (layer B.Cu) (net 4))
 (segment (start 140.5399 105.1) (end 138.9 106.7399) (width 0.3) (layer B.Cu) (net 4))
 (segment (start 138.9 106.7399) (end 138.9 107.4) (width 0.3) (layer B.Cu) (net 4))
 (segment (start 144.6739 76.7) (end 146.2748 76.7) (width 0.3) (layer B.Cu) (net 4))
 (segment (start 143.7742 73.3001) (end 143.7742 75.8003) (width 0.3) (layer B.Cu) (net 4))
 (segment (start 143.7742 75.8003) (end 144.6739 76.7) (width 0.3) (layer B.Cu) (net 4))
 (segment (start 144.6739 76.7) (end 144.6739 82.65) (width 0.3) (layer B.Cu) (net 4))
 (segment (start 147.0999 76.7) (end 146.2748 76.7) (width 0.3) (layer B.Cu) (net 4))
 (segment (start 144 73.3001) (end 143.7742 73.3001) (width 0.3) (layer B.Cu) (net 4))
 (segment (start 143.762 73.3001) (end 143.7742 73.3001) (width 0.3) (layer B.Cu) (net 4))
 (segment (start 143.762 73.3001) (end 143.1749 73.3001) (width 0.3) (layer B.Cu) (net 4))
 (segment (start 144.2 87.3) (end 144.2 83.1239) (width 0.3) (layer B.Cu) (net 4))
 (segment (start 144.2 83.1239) (end 144.6739 82.65) (width 0.3) (layer B.Cu) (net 4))
 (segment (start 142.7 88.8) (end 144.2 87.3) (width 0.3) (layer B.Cu) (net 4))
 (segment (start 145.574 82.65) (end 144.6739 82.65) (width 0.3) (layer B.Cu) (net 4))
 (segment (start 142.7 90.4) (end 142.7 88.8) (width 0.3) (layer B.Cu) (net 4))
 (segment (start 140.5 87.8699) (end 141.7699 87.8699) (width 0.3) (layer B.Cu) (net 4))
 (segment (start 141.7699 87.8699) (end 142.7 88.8) (width 0.3) (layer B.Cu) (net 4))
 (segment (start 140.5 87.8699) (end 140.5 87.5399) (width 0.3) (layer B.Cu) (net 4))
 (segment (start 140.5 88.2) (end 140.5 87.8699) (width 0.3) (layer B.Cu) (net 4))
 (segment (start 147.6251 83.3) (end 146.9751 82.65) (width 0.3) (layer B.Cu) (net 4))
 (segment (start 146.9751 82.65) (end 145.574 82.65) (width 0.3) (layer B.Cu) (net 4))
 (segment (start 147.6251 83.3) (end 148.0501 83.3) (width 0.3) (layer B.Cu) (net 4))
 (segment (start 147.2 83.3) (end 147.6251 83.3) (width 0.3) (layer B.Cu) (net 4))
 (segment (start 139.5 83.5) (end 139.5 84.4251) (width 0.3) (layer B.Cu) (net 4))
 (segment (start 141.53 99.4) (end 141.53 98.4999) (width 0.3) (layer B.Cu) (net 4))
 (segment (start 141.53 98.4999) (end 140.76 98.4999) (width 0.3) (layer B.Cu) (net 4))
 (segment (start 140.76 98.4999) (end 139.5601 97.3) (width 0.3) (layer B.Cu) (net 4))
 (segment (start 141.53 99.4) (end 141.53 100.3002) (width 0.3) (layer B.Cu) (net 4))
 (segment (start 138.9 97.3) (end 139.5601 97.3) (width 0.3) (layer B.Cu) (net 4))
 (segment (start 141.2 105.1) (end 140.5399 105.1) (width 0.3) (layer B.Cu) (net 4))
 (segment (start 141.53 103.2001) (end 141.2 103.5301) (width 0.3) (layer B.Cu) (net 4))
 (segment (start 141.2 103.5301) (end 141.2 105.1) (width 0.3) (layer B.Cu) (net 4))
 (segment (start 152.375 94.375) (end 152.375 89.625) (width 0.3) (layer B.Cu) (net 4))
 (segment (start 150.9 106.3399) (end 152.375 104.8649) (width 0.3) (layer B.Cu) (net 4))
 (segment (start 152.375 104.8649) (end 152.375 94.375) (width 0.3) (layer B.Cu) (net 4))
 (segment (start 141.3 83.3) (end 140.4499 83.3) (width 0.3) (layer B.Cu) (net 4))
 (segment (start 139.5 83.5) (end 140.2499 83.5) (width 0.3) (layer B.Cu) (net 4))
 (segment (start 140.2499 83.5) (end 140.4499 83.3) (width 0.3) (layer B.Cu) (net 4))
 (segment (start 149 83.5) (end 148.2501 83.5) (width 0.3) (layer B.Cu) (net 4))
 (segment (start 148.2501 83.5) (end 148.0501 83.3) (width 0.3) (layer B.Cu) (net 4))
 (segment (start 142.1 73.5) (end 142.975 73.5) (width 0.3) (layer B.Cu) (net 4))
 (segment (start 142.975 73.5) (end 143.1749 73.3001) (width 0.3) (layer B.Cu) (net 4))
 (segment (start 144.07 99.4) (end 144.07 98.4999) (width 0.3) (layer B.Cu) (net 4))
 (segment (start 148.2763 94.375) (end 144.1514 98.4999) (width 0.3) (layer B.Cu) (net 4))
 (segment (start 144.1514 98.4999) (end 144.07 98.4999) (width 0.3) (layer B.Cu) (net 4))
 (segment (start 148.2763 94.375) (end 148.9276 94.375) (width 0.3) (layer B.Cu) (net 4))
 (segment (start 147.625 94.375) (end 148.2763 94.375) (width 0.3) (layer B.Cu) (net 4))
 (segment (start 152.375 94.375) (end 148.9276 94.375) (width 0.3) (layer B.Cu) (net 4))
 (segment (start 147.625 89.625) (end 152.375 89.625) (width 0.3) (layer B.Cu) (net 4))
 (segment (start 144.07 100.3002) (end 144.07 101.85) (width 0.3) (layer B.Cu) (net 4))
 (segment (start 144.07 99.4) (end 144.07 100.3002) (width 0.3) (layer B.Cu) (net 4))
 (segment (start 144.07 100.3002) (end 141.53 100.3002) (width 0.3) (layer B.Cu) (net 4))
 (segment (start 141.53 100.3002) (end 141.53 102.3) (width 0.3) (layer B.Cu) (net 4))
 (segment (start 141.53 102.3) (end 141.53 103.2001) (width 0.3) (layer B.Cu) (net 4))
 (segment (start 144.2749 109.6) (end 145.1 109.6) (width 0.3) (layer B.Cu) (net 4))
 (segment (start 144.2749 109.6) (end 144.2749 108.95) (width 0.3) (layer B.Cu) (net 4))
 (segment (start 145.1 108.95) (end 144.2749 108.95) (width 0.3) (layer B.Cu) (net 4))
 (segment (start 138.3 92) (end 138.3 93.3749) (width 0.3) (layer B.Cu) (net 4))
 (segment (start 138.3 93.3749) (end 138.3 94.2) (width 0.3) (layer B.Cu) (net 4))
 (segment (start 138.3 93.3749) (end 138.95 93.3749) (width 0.3) (layer B.Cu) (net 4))
 (segment (start 138.95 94.2) (end 138.95 93.3749) (width 0.3) (layer B.Cu) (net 4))
 (segment (start 147.3398 74.56) (end 147.51 74.73) (width 0.6) (layer B.Cu) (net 17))
 (segment (start 147.012 73.075) (end 147.012 74.2325) (width 0.6) (layer B.Cu) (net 17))
 (segment (start 147.012 74.2325) (end 147.3398 74.56) (width 0.6) (layer B.Cu) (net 17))
 (segment (start 147.17 74.73) (end 147.3398 74.5602) (width 0.3) (layer B.Cu) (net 17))
 (segment (start 147.3398 74.5602) (end 147.3398 74.56) (width 0.3) (layer B.Cu) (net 17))
 (segment (start 152.83 74.73) (end 152.739 74.639) (width 0.3) (layer B.Cu) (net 17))
 (segment (start 152.739 74.639) (end 152.739 74.4812) (width 0.3) (layer B.Cu) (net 17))
 (segment (start 152.739 74.4812) (end 152.49 74.73) (width 0.6) (layer B.Cu) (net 17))
 (segment (start 152.988 73.075) (end 152.988 74.2325) (width 0.6) (layer B.Cu) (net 17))
 (segment (start 152.988 74.2325) (end 152.739 74.4812) (width 0.6) (layer B.Cu) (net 17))
 (segment (start 145.875 71.7) (end 145.95 71.7) (width 0.3) (layer B.Cu) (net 17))
 (segment (start 145.95 71.7) (end 146 71.65) (width 0.3) (layer B.Cu) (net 17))
 (segment (start 145.875 71.7) (end 144 71.7) (width 0.6) (layer B.Cu) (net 17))
 (segment (start 144 71.7) (end 144 71.6999) (width 0.6) (layer B.Cu) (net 17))
 (segment (start 154.125 71.8187) (end 154 71.6937) (width 0.3) (layer B.Cu) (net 17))
 (segment (start 154 71.6937) (end 154 71.65) (width 0.3) (layer B.Cu) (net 17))
 (segment (start 154.125 71.8187) (end 154.125 71.9375) (width 0.6) (layer B.Cu) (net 17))
 (segment (start 154.125 71.9375) (end 152.988 73.075) (width 0.6) (layer B.Cu) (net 17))
 (segment (start 154.125 71.7) (end 154.125 71.8187) (width 0.6) (layer B.Cu) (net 17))
 (segment (start 149.0625 71.45) (end 150.9375 71.45) (width 0.3) (layer B.Cu) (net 17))
 (segment (start 149.062 71.45) (end 149.0625 71.45) (width 0.3) (layer B.Cu) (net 17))
 (segment (start 150.9375 71.45) (end 150.938 71.45) (width 0.3) (layer B.Cu) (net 17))
 (segment (start 152.9875 73.075) (end 152.562 73.075) (width 0.6) (layer B.Cu) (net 17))
 (segment (start 152.562 73.075) (end 150.938 71.45) (width 0.6) (layer B.Cu) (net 17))
 (segment (start 152.988 73.075) (end 152.9875 73.075) (width 0.6) (layer B.Cu) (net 17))
 (segment (start 147.0125 73.075) (end 147.438 73.075) (width 0.6) (layer B.Cu) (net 17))
 (segment (start 147.438 73.075) (end 149.062 71.45) (width 0.6) (layer B.Cu) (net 17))
 (segment (start 147.012 73.075) (end 147.0125 73.075) (width 0.6) (layer B.Cu) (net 17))
 (segment (start 144 71.6999) (end 142.1 71.6999) (width 0.6) (layer B.Cu) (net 17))
 (segment (start 142.1 71.6999) (end 142.1 71.7) (width 0.6) (layer B.Cu) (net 17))
 (segment (start 145.875 71.7) (end 145.875 71.9375) (width 0.6) (layer B.Cu) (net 17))
 (segment (start 145.875 71.9375) (end 147.012 73.075) (width 0.6) (layer B.Cu) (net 17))
 (segment (start 138.0202 89.5202) (end 138.9 90.4) (width 0.3) (layer B.Cu) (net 6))
 (segment (start 139.8 108.0601) (end 138.4445 108.0601) (width 0.3) (layer B.Cu) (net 6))
 (segment (start 138.4445 108.0601) (end 136.443 106.0586) (width 0.3) (layer B.Cu) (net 6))
 (segment (start 136.443 106.0586) (end 136.443 89.8099) (width 0.3) (layer B.Cu) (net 6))
 (segment (start 136.443 89.8099) (end 136.7327 89.5202) (width 0.3) (layer B.Cu) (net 6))
 (segment (start 136.7327 89.5202) (end 138.0202 89.5202) (width 0.3) (layer B.Cu) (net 6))
 (segment (start 138.0202 89.5202) (end 138.0202 83.1798) (width 0.3) (layer B.Cu) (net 6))
 (segment (start 138.0202 83.1798) (end 139.5 81.7) (width 0.3) (layer B.Cu) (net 6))
 (segment (start 139.8 107.4) (end 139.8 108.0601) (width 0.3) (layer B.Cu) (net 6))
 (segment (start 141.3 81.7) (end 139.5 81.7) (width 0.3) (layer B.Cu) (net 6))
 (segment (start 138.9 90.4) (end 139.7001 90.4) (width 0.3) (layer B.Cu) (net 6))
 (segment (start 139.8 107.4) (end 141.1999 107.4) (width 0.3) (layer B.Cu) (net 6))
 (segment (start 140.5 90.3998) (end 139.7003 90.3998) (width 0.3) (layer B.Cu) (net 6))
 (segment (start 139.7003 90.3998) (end 139.7001 90.4) (width 0.3) (layer B.Cu) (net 6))
 (segment (start 140.5 89.1) (end 140.5 90.3998) (width 0.3) (layer B.Cu) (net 6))
 (segment (start 141.2 109) (end 141.2 108.1999) (width 0.3) (layer B.Cu) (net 6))
 (segment (start 141.1999 107.4) (end 141.1999 108.1999) (width 0.3) (layer B.Cu) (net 6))
 (segment (start 141.1999 108.1999) (end 141.2 108.1999) (width 0.3) (layer B.Cu) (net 6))
 (segment (start 141.3 81.7) (end 142.874 81.7) (width 0.3) (layer B.Cu) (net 6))
 (segment (start 140.5 90.3998) (end 141.3251 90.3998) (width 0.3) (layer B.Cu) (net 6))
 (segment (start 141.8 90.4) (end 141.3253 90.4) (width 0.3) (layer B.Cu) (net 6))
 (segment (start 141.3253 90.4) (end 141.3251 90.3998) (width 0.3) (layer B.Cu) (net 6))
 (segment (start 141.2 106) (end 141.2 106.6601) (width 0.3) (layer B.Cu) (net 6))
 (segment (start 141.2 106.6601) (end 141.1999 106.6601) (width 0.3) (layer B.Cu) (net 6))
 (segment (start 141.1999 106.6601) (end 141.1999 107.4) (width 0.3) (layer B.Cu) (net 6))
 (segment (start 142.8001 107.4001) (end 142.8001 107.4) (width 0.3) (layer B.Cu) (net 14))
 (segment (start 142.9 108.95) (end 142.9 107.5) (width 0.3) (layer B.Cu) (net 14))
 (segment (start 142.9 107.5) (end 142.8001 107.4001) (width 0.3) (layer B.Cu) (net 14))
 (segment (start 142.8001 107.4001) (end 142.8 107.4) (width 0.3) (layer B.Cu) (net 14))
 (segment (start 142.8 107.4) (end 142.8 106.1) (width 0.3) (layer B.Cu) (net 14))
 (segment (start 142.8 105.2) (end 142.8 102.3) (width 0.3) (layer B.Cu) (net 11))
 (segment (start 151.3 81.7) (end 151.3 78.3002) (width 0.6) (layer B.Cu) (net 3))
 (segment (start 146 85.4302) (end 150.07 85.4302) (width 0.6) (layer B.Cu) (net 3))
 (segment (start 150.07 85.4302) (end 151.3 84.2) (width 0.6) (layer B.Cu) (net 3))
 (segment (start 151.3 84.2) (end 151.3 81.7) (width 0.6) (layer B.Cu) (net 3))
 (segment (start 147.2 81.7) (end 149 81.7) (width 0.6) (layer B.Cu) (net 3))
 (segment (start 145.574 81.7) (end 147.2 81.7) (width 0.6) (layer B.Cu) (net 3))
 (segment (start 144.2 90.3998) (end 144.2 88.9) (width 0.6) (layer B.Cu) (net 3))
 (segment (start 144.2 88.9) (end 145.3 88.9) (width 0.6) (layer B.Cu) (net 3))
 (segment (start 145.3 88.9) (end 146 88.2) (width 0.6) (layer B.Cu) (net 3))
 (segment (start 146 88.2) (end 146 85.4302) (width 0.6) (layer B.Cu) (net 3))
 (segment (start 145.574 83.6) (end 145.574 85.004) (width 0.3) (layer B.Cu) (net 3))
 (segment (start 145.574 85.004) (end 146 85.4302) (width 0.3) (layer B.Cu) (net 3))
 (segment (start 149 81.7) (end 151.3 81.7) (width 0.6) (layer B.Cu) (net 3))
 (segment (start 142.8 96.4) (end 142.8 96.36) (width 0.3) (layer B.Cu) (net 10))
 (segment (start 142.8 99.4) (end 142.8 96.4) (width 0.3) (layer B.Cu) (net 10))
 (segment (start 141.9 96.4) (end 138.9 96.4) (width 0.3) (layer B.Cu) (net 21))
 (segment (start 138.9 96.4) (end 137.8 96.4) (width 0.3) (layer B.Cu) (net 21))
 (segment (start 140.5 92) (end 138.95 92) (width 0.3) (layer B.Cu) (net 13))
 (segment (start 140.5 92) (end 141.9 92) (width 0.3) (layer B.Cu) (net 13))
 (segment (start 142.8 92) (end 144.2 92) (width 0.3) (layer B.Cu) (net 7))
 (segment (start 144.2 92) (end 150 92) (width 0.3) (layer B.Cu) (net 7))
 (segment (start 148.7 76.13) (end 148.7001 76.1301) (width 0.3) (layer B.Cu) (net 16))
 (segment (start 148.7001 76.1301) (end 148.7001 76.7) (width 0.3) (layer B.Cu) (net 16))
 (segment (start 148.7 76.13) (end 148.7 76.7) (width 0.4) (layer B.Cu) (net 16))
 (segment (start 148.7 74.525) (end 148.7 76.13) (width 0.4) (layer B.Cu) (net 16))
 (segment (start 151.3 74.525) (end 151.3 76.7) (width 0.4) (layer B.Cu) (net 15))
 (segment (start 145.1 110.25) (end 149.75 110.25) (width 0.3) (layer B.Cu) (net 23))
 (segment (start 149.75 110.25) (end 150 110) (width 0.3) (layer B.Cu) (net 23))
 (segment (start 150 110) (end 150 109) (width 0.3) (layer B.Cu) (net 23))
 (segment (start 137.65 94.2) (end 137.65 95.29) (width 0.3) (layer B.Cu) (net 24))
 (segment (start 137.65 95.29) (end 137.8 95.44) (width 0.3) (layer B.Cu) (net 24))
 (segment (start 149.04 105.2) (end 143.76 105.2) (width 0.3) (layer B.Cu) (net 1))
 (segment (start 142.9 110.25) (end 141.55 110.25) (width 0.4) (layer B.Cu) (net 12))
 (segment (start 141.55 110.25) (end 141.2 110.6) (width 0.4) (layer B.Cu) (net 12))
 (segment (start 142.8 95.4) (end 142.8 92.96) (width 0.3) (layer B.Cu) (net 8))
 (segment (start 137.65 92) (end 137.65 90.75) (width 0.4) (layer B.Cu) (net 9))
 (segment (start 137.65 90.75) (end 137.3 90.4) (width 0.4) (layer B.Cu) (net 9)))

